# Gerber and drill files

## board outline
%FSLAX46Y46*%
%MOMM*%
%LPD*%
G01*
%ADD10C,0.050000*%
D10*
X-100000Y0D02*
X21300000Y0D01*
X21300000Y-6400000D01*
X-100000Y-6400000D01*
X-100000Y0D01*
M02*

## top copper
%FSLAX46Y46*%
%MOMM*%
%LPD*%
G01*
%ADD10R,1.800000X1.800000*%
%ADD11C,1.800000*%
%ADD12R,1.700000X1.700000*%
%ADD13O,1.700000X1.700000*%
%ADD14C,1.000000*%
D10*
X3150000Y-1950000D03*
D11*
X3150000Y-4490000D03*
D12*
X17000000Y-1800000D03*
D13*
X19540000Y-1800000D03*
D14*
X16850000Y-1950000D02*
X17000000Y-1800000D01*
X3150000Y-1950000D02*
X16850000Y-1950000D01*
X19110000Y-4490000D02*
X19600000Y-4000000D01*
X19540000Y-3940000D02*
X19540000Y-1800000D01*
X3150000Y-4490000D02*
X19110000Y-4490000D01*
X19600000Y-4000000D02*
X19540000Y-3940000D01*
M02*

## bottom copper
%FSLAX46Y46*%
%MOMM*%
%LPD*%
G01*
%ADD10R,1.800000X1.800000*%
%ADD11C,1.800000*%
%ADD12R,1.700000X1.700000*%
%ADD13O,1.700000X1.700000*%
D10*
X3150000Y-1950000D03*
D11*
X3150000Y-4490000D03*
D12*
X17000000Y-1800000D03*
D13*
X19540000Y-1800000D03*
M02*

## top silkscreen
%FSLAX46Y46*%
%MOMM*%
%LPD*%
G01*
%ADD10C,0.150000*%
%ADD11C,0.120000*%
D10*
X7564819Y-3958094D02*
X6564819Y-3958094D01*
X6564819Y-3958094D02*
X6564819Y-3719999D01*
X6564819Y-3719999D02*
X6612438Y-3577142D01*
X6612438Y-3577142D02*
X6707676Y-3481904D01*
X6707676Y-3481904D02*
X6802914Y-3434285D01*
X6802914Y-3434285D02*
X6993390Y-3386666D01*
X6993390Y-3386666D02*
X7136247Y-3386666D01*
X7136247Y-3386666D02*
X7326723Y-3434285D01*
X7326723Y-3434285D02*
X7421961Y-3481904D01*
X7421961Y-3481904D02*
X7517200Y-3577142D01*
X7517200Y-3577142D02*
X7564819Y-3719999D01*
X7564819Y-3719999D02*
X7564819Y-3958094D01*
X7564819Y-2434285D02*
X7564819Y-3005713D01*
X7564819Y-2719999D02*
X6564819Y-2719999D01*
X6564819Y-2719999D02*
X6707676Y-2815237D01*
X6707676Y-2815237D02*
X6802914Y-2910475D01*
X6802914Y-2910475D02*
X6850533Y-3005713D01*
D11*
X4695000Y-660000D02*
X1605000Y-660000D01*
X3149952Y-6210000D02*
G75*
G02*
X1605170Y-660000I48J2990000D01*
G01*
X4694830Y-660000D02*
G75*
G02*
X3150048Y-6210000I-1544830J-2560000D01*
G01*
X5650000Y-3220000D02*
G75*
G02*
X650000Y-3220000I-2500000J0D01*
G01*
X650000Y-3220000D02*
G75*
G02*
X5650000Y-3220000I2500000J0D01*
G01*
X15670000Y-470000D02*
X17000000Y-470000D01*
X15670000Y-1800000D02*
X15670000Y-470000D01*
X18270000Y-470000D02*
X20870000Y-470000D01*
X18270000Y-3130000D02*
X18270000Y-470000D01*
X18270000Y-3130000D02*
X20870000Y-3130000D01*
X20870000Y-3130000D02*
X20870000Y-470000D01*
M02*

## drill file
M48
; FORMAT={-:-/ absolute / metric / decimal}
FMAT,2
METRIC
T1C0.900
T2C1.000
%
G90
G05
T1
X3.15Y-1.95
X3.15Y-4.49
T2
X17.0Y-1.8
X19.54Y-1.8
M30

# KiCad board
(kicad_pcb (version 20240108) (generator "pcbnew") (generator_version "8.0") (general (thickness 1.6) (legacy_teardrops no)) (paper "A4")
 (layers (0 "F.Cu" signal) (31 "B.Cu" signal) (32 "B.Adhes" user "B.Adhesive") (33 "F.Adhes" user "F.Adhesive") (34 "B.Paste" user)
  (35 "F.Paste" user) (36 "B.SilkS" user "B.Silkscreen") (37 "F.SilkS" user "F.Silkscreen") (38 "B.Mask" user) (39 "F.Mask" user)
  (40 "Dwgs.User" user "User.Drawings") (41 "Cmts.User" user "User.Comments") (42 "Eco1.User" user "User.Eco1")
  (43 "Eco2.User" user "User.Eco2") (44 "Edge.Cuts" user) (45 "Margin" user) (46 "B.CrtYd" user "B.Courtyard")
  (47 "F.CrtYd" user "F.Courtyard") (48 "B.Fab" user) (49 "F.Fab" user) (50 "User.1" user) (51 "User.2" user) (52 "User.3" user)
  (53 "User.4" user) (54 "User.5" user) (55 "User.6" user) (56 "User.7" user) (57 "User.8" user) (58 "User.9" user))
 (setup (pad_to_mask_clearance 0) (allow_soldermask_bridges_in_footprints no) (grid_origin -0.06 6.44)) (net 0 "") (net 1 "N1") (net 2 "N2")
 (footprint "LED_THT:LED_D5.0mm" (layer "F.Cu") (at 3.15 1.95 -90)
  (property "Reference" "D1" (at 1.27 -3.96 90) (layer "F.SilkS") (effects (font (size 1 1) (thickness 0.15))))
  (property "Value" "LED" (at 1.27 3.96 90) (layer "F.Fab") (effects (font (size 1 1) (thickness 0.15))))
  (fp_line (start -1.29 -1.545) (end -1.29 1.545) (stroke (width 0.12) (type solid)) (layer "F.SilkS"))
  (fp_arc (start 4.26 0.000048) (mid 2.071756 2.880501) (end -1.29 1.54483) (stroke (width 0.12) (type solid)) (layer "F.SilkS"))
  (fp_arc (start -1.29 -1.54483) (mid 2.071756 -2.880501) (end 4.26 -0.000048) (stroke (width 0.12) (type solid)) (layer "F.SilkS"))
  (fp_circle (center 1.27 0) (end 3.77 0) (stroke (width 0.12) (type solid)) (fill none) (layer "F.SilkS"))
  (pad "1" thru_hole rect (at 0 0 270) (size 1.8 1.8) (drill 0.9) (layers "*.Cu" "*.Mask") (remove_unused_layers no) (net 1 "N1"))
  (pad "2" thru_hole circle (at 2.54 0 270) (size 1.8 1.8) (drill 0.9) (layers "*.Cu" "*.Mask") (remove_unused_layers no) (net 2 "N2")))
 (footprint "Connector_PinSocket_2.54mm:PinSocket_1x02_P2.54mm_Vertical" (layer "F.Cu") (at 17 1.8 90)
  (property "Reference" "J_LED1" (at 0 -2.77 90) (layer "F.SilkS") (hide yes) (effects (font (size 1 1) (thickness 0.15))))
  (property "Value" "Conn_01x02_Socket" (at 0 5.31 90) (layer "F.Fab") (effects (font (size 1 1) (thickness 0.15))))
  (fp_line (start 1.33 -1.33) (end 1.33 0) (stroke (width 0.12) (type solid)) (layer "F.SilkS"))
  (fp_line (start 0 -1.33) (end 1.33 -1.33) (stroke (width 0.12) (type solid)) (layer "F.SilkS"))
  (fp_line (start 1.33 1.27) (end 1.33 3.87) (stroke (width 0.12) (type solid)) (layer "F.SilkS"))
  (fp_line (start -1.33 1.27) (end 1.33 1.27) (stroke (width 0.12) (type solid)) (layer "F.SilkS"))
  (fp_line (start -1.33 1.27) (end -1.33 3.87) (stroke (width 0.12) (type solid)) (layer "F.SilkS"))
  (fp_line (start -1.33 3.87) (end 1.33 3.87) (stroke (width 0.12) (type solid)) (layer "F.SilkS"))
  (pad "1" thru_hole rect (at 0 0 90) (size 1.7 1.7) (drill 1) (layers "*.Cu" "*.Mask") (remove_unused_layers no) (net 1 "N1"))
  (pad "2" thru_hole oval (at 0 2.54 90) (size 1.7 1.7) (drill 1) (layers "*.Cu" "*.Mask") (remove_unused_layers no) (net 2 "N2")))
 (gr_rect (start -0.1 0) (end 21.3 6.4) (stroke (width 0.05) (type default)) (fill none) (layer "Edge.Cuts"))
 (segment (start 16.85 1.95) (end 17 1.8) (width 1) (layer "F.Cu") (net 1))
 (segment (start 3.15 1.95) (end 16.85 1.95) (width 1) (layer "F.Cu") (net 1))
 (segment (start 19.11 4.49) (end 19.6 4) (width 1) (layer "F.Cu") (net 2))
 (segment (start 19.54 3.94) (end 19.54 1.8) (width 1) (layer "F.Cu") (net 2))
 (segment (start 3.15 4.49) (end 19.11 4.49) (width 1) (layer "F.Cu") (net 2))
 (segment (start 19.6 4) (end 19.54 3.94) (width 1) (layer "F.Cu") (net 2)))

